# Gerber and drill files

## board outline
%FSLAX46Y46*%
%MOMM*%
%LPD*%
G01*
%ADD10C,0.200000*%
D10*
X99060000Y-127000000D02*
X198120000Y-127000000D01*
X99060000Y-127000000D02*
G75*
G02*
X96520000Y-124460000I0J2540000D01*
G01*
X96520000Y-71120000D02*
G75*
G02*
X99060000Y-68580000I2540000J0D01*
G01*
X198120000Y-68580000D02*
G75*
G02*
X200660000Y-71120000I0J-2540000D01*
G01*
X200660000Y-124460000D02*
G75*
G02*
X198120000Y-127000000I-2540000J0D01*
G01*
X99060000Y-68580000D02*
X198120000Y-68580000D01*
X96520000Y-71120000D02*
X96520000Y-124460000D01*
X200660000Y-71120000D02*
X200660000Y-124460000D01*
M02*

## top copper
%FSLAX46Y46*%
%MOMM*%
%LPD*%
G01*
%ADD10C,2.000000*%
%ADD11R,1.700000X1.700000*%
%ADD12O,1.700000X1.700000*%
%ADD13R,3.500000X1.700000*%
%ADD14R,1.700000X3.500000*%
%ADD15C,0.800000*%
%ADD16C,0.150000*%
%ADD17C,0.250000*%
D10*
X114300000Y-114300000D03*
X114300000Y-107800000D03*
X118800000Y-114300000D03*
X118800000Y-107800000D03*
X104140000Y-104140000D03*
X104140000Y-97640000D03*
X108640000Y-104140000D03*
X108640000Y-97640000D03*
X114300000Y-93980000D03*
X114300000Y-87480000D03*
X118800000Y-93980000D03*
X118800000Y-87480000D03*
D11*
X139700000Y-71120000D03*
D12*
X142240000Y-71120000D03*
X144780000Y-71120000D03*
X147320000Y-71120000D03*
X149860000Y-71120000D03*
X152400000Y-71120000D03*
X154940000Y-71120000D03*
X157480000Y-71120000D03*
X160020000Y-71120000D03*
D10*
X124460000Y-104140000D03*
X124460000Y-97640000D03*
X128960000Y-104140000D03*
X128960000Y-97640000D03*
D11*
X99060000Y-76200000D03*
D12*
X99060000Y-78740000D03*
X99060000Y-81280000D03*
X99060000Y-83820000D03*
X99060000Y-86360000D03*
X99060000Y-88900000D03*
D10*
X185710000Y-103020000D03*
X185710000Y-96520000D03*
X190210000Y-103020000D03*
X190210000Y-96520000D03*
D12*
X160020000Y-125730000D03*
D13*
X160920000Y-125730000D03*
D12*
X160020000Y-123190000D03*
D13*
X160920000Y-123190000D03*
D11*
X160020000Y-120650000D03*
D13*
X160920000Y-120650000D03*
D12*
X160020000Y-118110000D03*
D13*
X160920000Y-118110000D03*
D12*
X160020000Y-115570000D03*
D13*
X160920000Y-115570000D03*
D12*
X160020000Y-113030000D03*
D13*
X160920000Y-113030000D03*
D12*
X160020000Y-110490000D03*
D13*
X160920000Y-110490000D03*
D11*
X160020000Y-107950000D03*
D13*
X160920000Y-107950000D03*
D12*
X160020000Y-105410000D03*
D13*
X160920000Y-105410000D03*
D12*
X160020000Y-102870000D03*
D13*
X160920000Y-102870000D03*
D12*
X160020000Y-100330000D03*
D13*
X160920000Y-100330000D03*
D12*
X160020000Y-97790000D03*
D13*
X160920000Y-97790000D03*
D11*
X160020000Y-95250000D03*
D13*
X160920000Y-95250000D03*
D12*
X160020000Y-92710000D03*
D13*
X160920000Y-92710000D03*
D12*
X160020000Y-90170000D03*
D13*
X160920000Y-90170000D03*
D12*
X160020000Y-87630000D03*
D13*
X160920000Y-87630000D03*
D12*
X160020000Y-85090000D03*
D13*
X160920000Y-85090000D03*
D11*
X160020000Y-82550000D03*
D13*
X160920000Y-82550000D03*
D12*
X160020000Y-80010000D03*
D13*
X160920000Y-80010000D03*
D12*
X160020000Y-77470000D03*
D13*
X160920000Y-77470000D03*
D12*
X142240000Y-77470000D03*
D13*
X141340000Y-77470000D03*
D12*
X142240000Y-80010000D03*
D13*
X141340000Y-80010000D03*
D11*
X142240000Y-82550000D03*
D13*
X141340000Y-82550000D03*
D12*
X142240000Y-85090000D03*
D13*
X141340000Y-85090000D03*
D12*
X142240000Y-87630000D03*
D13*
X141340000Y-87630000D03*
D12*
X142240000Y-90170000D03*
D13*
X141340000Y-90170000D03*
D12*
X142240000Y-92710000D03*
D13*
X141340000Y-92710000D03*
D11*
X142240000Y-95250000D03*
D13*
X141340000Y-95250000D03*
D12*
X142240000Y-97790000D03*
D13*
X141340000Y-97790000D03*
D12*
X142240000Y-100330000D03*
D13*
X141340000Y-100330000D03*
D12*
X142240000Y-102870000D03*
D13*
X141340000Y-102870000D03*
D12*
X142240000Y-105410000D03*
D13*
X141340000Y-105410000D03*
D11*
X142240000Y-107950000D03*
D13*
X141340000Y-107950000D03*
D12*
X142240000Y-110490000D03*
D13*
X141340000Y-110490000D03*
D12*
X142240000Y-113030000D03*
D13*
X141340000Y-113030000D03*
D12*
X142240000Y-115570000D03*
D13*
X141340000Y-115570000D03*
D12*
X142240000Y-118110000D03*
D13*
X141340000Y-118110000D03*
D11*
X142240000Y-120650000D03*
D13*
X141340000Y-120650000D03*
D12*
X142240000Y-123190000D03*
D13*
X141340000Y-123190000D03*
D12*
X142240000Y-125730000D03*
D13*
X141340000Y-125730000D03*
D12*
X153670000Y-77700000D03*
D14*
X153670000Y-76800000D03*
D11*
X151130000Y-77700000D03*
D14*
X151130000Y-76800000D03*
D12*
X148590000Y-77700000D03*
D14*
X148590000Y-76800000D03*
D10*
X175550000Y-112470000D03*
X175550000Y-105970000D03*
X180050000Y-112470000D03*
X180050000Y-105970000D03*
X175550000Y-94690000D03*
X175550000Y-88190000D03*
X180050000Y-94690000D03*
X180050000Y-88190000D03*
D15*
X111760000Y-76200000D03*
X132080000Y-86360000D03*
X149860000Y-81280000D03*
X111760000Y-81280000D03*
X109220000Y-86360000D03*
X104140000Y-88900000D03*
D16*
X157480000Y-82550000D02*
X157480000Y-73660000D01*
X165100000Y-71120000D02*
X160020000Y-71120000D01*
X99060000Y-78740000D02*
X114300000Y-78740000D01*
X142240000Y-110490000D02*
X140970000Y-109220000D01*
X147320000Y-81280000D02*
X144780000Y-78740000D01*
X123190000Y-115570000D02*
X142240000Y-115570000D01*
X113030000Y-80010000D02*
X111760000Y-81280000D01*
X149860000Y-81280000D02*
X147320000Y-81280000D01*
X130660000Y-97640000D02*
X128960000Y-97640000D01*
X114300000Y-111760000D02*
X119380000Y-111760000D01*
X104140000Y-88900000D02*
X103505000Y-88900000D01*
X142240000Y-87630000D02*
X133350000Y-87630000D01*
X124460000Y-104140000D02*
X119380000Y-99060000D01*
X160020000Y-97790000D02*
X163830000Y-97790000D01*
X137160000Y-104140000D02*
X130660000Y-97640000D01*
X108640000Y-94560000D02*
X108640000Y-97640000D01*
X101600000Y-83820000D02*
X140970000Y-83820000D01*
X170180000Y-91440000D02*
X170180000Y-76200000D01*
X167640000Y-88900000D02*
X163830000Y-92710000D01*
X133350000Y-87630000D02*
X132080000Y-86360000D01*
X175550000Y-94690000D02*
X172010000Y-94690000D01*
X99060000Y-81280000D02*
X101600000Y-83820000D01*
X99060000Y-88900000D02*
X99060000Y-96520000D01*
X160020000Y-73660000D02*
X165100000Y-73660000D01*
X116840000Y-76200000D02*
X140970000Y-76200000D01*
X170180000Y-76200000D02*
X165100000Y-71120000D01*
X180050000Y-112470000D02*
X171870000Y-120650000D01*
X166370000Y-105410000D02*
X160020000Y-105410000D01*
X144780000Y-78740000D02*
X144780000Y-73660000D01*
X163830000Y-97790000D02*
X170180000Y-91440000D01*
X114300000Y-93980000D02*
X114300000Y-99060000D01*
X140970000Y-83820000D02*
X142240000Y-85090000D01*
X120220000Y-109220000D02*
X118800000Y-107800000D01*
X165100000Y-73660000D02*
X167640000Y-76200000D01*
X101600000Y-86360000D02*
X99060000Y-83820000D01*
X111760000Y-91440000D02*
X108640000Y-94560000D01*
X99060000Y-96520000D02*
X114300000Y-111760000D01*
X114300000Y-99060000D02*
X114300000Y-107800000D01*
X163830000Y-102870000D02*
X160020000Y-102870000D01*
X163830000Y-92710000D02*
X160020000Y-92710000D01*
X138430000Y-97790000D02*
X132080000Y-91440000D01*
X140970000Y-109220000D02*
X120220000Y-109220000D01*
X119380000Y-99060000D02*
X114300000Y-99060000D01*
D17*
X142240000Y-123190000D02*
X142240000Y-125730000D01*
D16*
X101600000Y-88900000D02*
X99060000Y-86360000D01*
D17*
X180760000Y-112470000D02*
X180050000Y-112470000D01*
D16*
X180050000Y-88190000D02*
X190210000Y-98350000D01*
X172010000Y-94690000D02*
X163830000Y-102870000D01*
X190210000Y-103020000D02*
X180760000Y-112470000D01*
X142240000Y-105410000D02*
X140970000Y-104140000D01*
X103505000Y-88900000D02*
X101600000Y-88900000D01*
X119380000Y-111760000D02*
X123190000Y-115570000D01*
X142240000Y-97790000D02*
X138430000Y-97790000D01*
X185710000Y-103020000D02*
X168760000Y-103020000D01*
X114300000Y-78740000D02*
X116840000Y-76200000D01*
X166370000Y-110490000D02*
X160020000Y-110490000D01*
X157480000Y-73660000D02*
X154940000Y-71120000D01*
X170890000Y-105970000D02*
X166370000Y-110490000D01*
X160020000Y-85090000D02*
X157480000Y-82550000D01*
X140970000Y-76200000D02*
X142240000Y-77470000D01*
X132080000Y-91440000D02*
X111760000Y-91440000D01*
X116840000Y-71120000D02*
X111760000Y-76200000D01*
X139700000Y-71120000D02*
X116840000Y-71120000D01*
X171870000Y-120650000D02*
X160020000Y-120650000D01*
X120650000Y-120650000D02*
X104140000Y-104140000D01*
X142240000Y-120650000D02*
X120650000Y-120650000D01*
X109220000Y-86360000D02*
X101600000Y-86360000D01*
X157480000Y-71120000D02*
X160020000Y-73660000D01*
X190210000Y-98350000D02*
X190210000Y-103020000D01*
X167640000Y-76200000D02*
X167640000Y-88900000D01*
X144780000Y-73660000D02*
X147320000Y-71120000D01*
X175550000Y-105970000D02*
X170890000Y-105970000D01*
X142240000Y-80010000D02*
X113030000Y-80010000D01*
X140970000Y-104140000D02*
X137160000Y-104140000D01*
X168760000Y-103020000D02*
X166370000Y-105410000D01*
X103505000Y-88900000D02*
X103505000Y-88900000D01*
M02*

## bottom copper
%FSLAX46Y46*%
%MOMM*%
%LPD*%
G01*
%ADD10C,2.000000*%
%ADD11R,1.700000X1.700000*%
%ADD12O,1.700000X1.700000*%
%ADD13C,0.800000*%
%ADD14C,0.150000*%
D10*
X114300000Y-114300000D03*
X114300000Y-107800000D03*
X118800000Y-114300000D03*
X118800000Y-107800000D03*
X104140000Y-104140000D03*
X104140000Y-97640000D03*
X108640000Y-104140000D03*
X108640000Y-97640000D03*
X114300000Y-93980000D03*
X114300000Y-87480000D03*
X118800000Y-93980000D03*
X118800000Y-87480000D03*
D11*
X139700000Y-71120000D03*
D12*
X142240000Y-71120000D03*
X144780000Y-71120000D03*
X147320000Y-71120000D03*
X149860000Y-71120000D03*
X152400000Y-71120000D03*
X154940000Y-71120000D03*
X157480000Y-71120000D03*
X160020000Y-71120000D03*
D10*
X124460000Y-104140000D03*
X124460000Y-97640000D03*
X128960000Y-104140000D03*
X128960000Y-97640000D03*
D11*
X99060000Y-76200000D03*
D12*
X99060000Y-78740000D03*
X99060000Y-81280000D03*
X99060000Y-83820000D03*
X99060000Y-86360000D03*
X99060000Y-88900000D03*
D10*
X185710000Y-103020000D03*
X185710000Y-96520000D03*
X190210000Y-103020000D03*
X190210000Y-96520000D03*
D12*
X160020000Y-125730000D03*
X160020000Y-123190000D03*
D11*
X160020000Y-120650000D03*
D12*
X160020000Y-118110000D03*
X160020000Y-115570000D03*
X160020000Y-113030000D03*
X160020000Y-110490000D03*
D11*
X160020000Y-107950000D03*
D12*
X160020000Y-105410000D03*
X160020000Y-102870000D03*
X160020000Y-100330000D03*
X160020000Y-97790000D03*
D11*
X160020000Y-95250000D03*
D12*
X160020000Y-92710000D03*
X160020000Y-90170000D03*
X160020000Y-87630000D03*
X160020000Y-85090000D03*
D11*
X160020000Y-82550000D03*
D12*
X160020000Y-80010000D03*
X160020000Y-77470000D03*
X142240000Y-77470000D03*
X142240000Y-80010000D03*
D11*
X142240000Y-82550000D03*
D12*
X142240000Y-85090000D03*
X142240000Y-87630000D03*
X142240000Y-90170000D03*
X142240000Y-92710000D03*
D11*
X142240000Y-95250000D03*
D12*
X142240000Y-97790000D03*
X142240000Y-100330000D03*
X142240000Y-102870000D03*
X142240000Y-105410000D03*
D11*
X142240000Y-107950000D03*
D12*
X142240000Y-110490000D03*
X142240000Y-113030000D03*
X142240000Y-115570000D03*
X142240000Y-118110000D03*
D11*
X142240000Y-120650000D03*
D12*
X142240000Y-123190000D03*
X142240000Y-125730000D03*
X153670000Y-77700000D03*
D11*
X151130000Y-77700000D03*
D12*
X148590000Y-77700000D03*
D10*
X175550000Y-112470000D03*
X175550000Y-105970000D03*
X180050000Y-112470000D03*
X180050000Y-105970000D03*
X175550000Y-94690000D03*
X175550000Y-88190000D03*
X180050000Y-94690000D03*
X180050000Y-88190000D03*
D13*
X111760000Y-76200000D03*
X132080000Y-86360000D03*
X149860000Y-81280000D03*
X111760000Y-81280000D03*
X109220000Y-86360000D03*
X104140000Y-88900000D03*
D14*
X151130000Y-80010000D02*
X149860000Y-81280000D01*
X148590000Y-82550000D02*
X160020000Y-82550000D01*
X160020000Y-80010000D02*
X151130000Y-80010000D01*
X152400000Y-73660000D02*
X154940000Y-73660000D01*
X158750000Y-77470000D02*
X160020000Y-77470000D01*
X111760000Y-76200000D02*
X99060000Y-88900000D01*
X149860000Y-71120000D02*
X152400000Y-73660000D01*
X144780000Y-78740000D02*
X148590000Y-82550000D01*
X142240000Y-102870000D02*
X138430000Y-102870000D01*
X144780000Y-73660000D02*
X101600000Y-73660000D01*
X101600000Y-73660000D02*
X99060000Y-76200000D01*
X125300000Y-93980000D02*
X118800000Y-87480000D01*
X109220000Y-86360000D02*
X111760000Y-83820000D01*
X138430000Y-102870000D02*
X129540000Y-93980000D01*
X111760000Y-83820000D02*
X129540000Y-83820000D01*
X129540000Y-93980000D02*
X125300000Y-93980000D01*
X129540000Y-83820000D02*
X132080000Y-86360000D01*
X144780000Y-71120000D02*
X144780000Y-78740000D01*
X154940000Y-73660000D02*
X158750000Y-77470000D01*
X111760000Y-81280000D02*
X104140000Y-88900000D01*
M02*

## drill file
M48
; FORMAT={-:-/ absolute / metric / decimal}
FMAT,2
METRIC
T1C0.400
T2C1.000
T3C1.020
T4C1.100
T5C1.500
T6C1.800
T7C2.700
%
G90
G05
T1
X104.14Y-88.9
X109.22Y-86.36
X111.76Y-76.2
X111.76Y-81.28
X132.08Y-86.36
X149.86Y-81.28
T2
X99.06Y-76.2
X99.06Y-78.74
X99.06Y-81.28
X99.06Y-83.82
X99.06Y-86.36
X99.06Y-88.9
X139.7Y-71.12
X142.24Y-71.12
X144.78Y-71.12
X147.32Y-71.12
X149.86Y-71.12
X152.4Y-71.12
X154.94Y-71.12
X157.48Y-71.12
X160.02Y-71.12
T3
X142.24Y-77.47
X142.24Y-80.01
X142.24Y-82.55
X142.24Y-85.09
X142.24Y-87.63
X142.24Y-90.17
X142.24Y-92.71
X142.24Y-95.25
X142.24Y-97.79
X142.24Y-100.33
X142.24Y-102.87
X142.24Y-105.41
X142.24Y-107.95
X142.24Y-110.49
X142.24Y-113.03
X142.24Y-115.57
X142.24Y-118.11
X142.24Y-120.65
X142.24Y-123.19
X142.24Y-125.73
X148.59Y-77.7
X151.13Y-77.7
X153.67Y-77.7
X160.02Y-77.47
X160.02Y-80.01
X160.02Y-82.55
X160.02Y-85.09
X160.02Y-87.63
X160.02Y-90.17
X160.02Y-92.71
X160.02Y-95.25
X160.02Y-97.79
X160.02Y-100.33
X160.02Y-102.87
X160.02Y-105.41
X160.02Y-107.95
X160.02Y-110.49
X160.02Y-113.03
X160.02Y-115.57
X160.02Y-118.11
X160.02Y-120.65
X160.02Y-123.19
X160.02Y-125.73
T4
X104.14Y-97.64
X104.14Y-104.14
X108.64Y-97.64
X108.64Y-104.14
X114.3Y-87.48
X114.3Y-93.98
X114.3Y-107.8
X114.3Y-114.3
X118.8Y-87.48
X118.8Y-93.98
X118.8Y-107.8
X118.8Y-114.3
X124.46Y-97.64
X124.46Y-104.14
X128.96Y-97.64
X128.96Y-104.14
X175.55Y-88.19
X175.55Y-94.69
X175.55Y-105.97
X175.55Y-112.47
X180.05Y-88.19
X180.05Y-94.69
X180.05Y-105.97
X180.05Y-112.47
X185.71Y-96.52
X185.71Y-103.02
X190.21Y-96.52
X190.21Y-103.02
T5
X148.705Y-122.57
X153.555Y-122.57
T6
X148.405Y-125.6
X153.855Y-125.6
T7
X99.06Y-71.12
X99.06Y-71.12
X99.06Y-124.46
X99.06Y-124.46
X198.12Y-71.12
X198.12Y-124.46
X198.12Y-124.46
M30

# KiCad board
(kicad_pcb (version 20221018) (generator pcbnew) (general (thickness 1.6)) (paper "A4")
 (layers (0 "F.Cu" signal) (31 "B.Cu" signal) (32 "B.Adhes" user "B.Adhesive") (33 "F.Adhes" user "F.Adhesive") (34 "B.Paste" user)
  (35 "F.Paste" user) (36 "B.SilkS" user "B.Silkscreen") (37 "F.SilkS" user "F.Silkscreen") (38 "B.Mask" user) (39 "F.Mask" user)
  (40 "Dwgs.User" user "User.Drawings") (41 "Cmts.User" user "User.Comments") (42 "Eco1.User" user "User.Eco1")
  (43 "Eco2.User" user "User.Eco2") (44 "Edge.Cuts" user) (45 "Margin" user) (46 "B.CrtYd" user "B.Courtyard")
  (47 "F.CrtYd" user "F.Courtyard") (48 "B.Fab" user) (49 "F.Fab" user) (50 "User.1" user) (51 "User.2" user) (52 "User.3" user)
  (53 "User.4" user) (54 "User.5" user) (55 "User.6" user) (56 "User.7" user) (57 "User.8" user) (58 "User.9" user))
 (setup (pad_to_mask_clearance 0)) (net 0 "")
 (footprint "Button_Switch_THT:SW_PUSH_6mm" (layer "F.Cu") (at 114.3 114.3 90)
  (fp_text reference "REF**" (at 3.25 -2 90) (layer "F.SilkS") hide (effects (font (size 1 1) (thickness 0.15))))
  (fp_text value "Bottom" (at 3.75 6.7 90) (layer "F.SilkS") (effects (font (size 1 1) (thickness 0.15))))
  (pad "1" thru_hole circle (at 0 0 180) (size 2 2) (drill 1.1) (layers "*.Cu" "*.Mask"))
  (pad "1" thru_hole circle (at 6.5 0 180) (size 2 2) (drill 1.1) (layers "*.Cu" "*.Mask"))
  (pad "2" thru_hole circle (at 0 4.5 180) (size 2 2) (drill 1.1) (layers "*.Cu" "*.Mask"))
  (pad "2" thru_hole circle (at 6.5 4.5 180) (size 2 2) (drill 1.1) (layers "*.Cu" "*.Mask")))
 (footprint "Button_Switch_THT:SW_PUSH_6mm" (layer "F.Cu") (at 104.14 104.14 90)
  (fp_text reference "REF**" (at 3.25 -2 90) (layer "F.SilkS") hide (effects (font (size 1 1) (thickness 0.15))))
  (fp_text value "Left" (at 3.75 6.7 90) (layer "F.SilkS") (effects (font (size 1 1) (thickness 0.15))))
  (pad "1" thru_hole circle (at 0 0 180) (size 2 2) (drill 1.1) (layers "*.Cu" "*.Mask"))
  (pad "1" thru_hole circle (at 6.5 0 180) (size 2 2) (drill 1.1) (layers "*.Cu" "*.Mask"))
  (pad "2" thru_hole circle (at 0 4.5 180) (size 2 2) (drill 1.1) (layers "*.Cu" "*.Mask"))
  (pad "2" thru_hole circle (at 6.5 4.5 180) (size 2 2) (drill 1.1) (layers "*.Cu" "*.Mask")))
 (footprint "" (layer "F.Cu") (at 198.12 71.12)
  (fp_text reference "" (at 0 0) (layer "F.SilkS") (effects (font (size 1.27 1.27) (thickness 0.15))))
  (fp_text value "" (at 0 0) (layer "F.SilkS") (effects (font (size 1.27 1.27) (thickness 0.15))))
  (pad "" np_thru_hole circle (at 0 0) (size 2.7 2.7) (drill 2.7) (layers "F&B.Cu" "*.Mask")))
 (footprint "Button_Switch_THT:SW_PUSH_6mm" (layer "F.Cu") (at 114.3 93.98 90)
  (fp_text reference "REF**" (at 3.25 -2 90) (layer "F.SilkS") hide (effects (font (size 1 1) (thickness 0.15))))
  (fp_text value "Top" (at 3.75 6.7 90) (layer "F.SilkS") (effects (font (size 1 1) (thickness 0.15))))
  (pad "1" thru_hole circle (at 0 0 180) (size 2 2) (drill 1.1) (layers "*.Cu" "*.Mask"))
  (pad "1" thru_hole circle (at 6.5 0 180) (size 2 2) (drill 1.1) (layers "*.Cu" "*.Mask"))
  (pad "2" thru_hole circle (at 0 4.5 180) (size 2 2) (drill 1.1) (layers "*.Cu" "*.Mask"))
  (pad "2" thru_hole circle (at 6.5 4.5 180) (size 2 2) (drill 1.1) (layers "*.Cu" "*.Mask")))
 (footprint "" (layer "F.Cu") (at 99.06 71.12)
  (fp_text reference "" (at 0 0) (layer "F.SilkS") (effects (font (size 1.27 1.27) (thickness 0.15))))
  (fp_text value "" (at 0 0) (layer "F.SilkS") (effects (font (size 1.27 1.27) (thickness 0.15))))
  (pad "" np_thru_hole circle (at 0 0) (size 2.7 2.7) (drill 2.7) (layers "F&B.Cu" "*.Mask")))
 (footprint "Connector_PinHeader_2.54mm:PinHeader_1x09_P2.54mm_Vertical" (layer "F.Cu") (at 139.7 71.12 90)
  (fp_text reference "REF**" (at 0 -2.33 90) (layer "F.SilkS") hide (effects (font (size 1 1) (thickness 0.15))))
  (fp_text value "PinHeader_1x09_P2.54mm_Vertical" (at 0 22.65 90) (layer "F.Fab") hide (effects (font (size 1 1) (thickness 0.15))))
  (pad "1" thru_hole rect (at 0 0 90) (size 1.7 1.7) (drill 1) (layers "*.Cu" "*.Mask"))
  (pad "2" thru_hole oval (at 0 2.54 90) (size 1.7 1.7) (drill 1) (layers "*.Cu" "*.Mask"))
  (pad "3" thru_hole oval (at 0 5.08 90) (size 1.7 1.7) (drill 1) (layers "*.Cu" "*.Mask"))
  (pad "4" thru_hole oval (at 0 7.62 90) (size 1.7 1.7) (drill 1) (layers "*.Cu" "*.Mask"))
  (pad "5" thru_hole oval (at 0 10.16 90) (size 1.7 1.7) (drill 1) (layers "*.Cu" "*.Mask"))
  (pad "6" thru_hole oval (at 0 12.7 90) (size 1.7 1.7) (drill 1) (layers "*.Cu" "*.Mask"))
  (pad "7" thru_hole oval (at 0 15.24 90) (size 1.7 1.7) (drill 1) (layers "*.Cu" "*.Mask"))
  (pad "8" thru_hole oval (at 0 17.78 90) (size 1.7 1.7) (drill 1) (layers "*.Cu" "*.Mask"))
  (pad "9" thru_hole oval (at 0 20.32 90) (size 1.7 1.7) (drill 1) (layers "*.Cu" "*.Mask")))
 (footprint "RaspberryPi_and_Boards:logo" (layer "F.Cu") (at 190.5 76.2)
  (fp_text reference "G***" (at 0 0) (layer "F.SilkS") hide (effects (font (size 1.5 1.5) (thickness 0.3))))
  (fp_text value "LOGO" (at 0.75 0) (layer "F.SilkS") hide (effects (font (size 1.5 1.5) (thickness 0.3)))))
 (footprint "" (layer "F.Cu") (at 198.12 124.46)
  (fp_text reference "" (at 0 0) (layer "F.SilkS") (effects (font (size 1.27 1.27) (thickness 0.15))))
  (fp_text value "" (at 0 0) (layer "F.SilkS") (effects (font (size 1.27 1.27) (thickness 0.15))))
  (pad "" np_thru_hole circle (at 0 0) (size 2.7 2.7) (drill 2.7) (layers "F&B.Cu" "*.Mask")))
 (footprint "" (layer "F.Cu") (at 198.12 124.46)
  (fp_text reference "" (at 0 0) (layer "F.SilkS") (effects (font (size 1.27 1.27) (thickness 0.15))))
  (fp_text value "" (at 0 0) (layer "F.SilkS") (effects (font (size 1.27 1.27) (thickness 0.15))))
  (pad "" np_thru_hole circle (at 0 0) (size 2.7 2.7) (drill 2.7) (layers "F&B.Cu" "*.Mask")))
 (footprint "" (layer "F.Cu") (at 99.06 124.46)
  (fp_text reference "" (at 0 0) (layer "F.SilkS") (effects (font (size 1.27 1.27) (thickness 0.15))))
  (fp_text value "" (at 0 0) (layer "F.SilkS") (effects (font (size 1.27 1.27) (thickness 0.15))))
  (pad "" np_thru_hole circle (at 0 0) (size 2.7 2.7) (drill 2.7) (layers "F&B.Cu" "*.Mask")))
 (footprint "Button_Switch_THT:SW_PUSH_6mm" (layer "F.Cu") (at 124.46 104.14 90)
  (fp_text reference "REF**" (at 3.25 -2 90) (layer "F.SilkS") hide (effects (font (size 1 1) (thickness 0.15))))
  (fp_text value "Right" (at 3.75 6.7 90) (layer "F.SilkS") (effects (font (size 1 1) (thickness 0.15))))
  (pad "1" thru_hole circle (at 0 0 180) (size 2 2) (drill 1.1) (layers "*.Cu" "*.Mask"))
  (pad "1" thru_hole circle (at 6.5 0 180) (size 2 2) (drill 1.1) (layers "*.Cu" "*.Mask"))
  (pad "2" thru_hole circle (at 0 4.5 180) (size 2 2) (drill 1.1) (layers "*.Cu" "*.Mask"))
  (pad "2" thru_hole circle (at 6.5 4.5 180) (size 2 2) (drill 1.1) (layers "*.Cu" "*.Mask")))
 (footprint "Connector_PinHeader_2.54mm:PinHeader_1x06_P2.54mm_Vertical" (layer "F.Cu") (at 99.06 76.2)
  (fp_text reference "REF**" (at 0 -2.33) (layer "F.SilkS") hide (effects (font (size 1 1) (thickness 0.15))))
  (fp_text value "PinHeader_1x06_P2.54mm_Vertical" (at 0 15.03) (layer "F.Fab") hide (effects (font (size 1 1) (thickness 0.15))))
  (pad "1" thru_hole rect (at 0 0) (size 1.7 1.7) (drill 1) (layers "*.Cu" "*.Mask"))
  (pad "2" thru_hole oval (at 0 2.54) (size 1.7 1.7) (drill 1) (layers "*.Cu" "*.Mask"))
  (pad "3" thru_hole oval (at 0 5.08) (size 1.7 1.7) (drill 1) (layers "*.Cu" "*.Mask"))
  (pad "4" thru_hole oval (at 0 7.62) (size 1.7 1.7) (drill 1) (layers "*.Cu" "*.Mask"))
  (pad "5" thru_hole oval (at 0 10.16) (size 1.7 1.7) (drill 1) (layers "*.Cu" "*.Mask"))
  (pad "6" thru_hole oval (at 0 12.7) (size 1.7 1.7) (drill 1) (layers "*.Cu" "*.Mask")))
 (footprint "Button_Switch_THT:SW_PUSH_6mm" (layer "F.Cu") (at 185.71 103.02 90)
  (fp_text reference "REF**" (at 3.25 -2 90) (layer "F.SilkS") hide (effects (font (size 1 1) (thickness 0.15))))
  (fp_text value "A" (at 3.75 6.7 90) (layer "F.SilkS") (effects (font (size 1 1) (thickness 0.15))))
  (pad "1" thru_hole circle (at 0 0 180) (size 2 2) (drill 1.1) (layers "*.Cu" "*.Mask"))
  (pad "1" thru_hole circle (at 6.5 0 180) (size 2 2) (drill 1.1) (layers "*.Cu" "*.Mask"))
  (pad "2" thru_hole circle (at 0 4.5 180) (size 2 2) (drill 1.1) (layers "*.Cu" "*.Mask"))
  (pad "2" thru_hole circle (at 6.5 4.5 180) (size 2 2) (drill 1.1) (layers "*.Cu" "*.Mask")))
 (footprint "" (layer "F.Cu") (at 99.06 124.46)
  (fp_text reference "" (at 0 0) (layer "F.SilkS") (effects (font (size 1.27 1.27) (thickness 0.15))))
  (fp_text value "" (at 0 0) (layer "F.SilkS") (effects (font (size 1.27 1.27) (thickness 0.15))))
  (pad "" np_thru_hole circle (at 0 0) (size 2.7 2.7) (drill 2.7) (layers "F&B.Cu" "*.Mask")))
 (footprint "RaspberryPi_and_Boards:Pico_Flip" (layer "F.Cu") (at 151.13 101.6 180)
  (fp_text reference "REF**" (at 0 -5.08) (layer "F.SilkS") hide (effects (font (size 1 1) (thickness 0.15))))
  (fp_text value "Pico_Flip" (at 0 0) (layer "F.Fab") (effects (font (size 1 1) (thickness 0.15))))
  (pad "" np_thru_hole oval (at -2.725 -24 180) (size 1.8 1.8) (drill 1.8) (layers "*.Cu" "*.Mask"))
  (pad "" np_thru_hole oval (at -2.425 -20.97 180) (size 1.5 1.5) (drill 1.5) (layers "*.Cu" "*.Mask"))
  (pad "" np_thru_hole oval (at 2.425 -20.97 180) (size 1.5 1.5) (drill 1.5) (layers "*.Cu" "*.Mask"))
  (pad "" np_thru_hole oval (at 2.725 -24 180) (size 1.8 1.8) (drill 1.8) (layers "*.Cu" "*.Mask"))
  (pad "1" thru_hole oval (at -8.89 -24.13 180) (size 1.7 1.7) (drill 1.02) (layers "*.Cu" "*.Mask"))
  (pad "1" smd rect (at -8.89 -24.13 180) (size 3.5 1.7) (drill (offset -0.9 0)) (layers "F.Cu" "F.Mask"))
  (pad "2" thru_hole oval (at -8.89 -21.59 180) (size 1.7 1.7) (drill 1.02) (layers "*.Cu" "*.Mask"))
  (pad "2" smd rect (at -8.89 -21.59 180) (size 3.5 1.7) (drill (offset -0.9 0)) (layers "F.Cu" "F.Mask"))
  (pad "3" thru_hole rect (at -8.89 -19.05 180) (size 1.7 1.7) (drill 1.02) (layers "*.Cu" "*.Mask"))
  (pad "3" smd rect (at -8.89 -19.05 180) (size 3.5 1.7) (drill (offset -0.9 0)) (layers "F.Cu" "F.Mask"))
  (pad "4" thru_hole oval (at -8.89 -16.51 180) (size 1.7 1.7) (drill 1.02) (layers "*.Cu" "*.Mask"))
  (pad "4" smd rect (at -8.89 -16.51 180) (size 3.5 1.7) (drill (offset -0.9 0)) (layers "F.Cu" "F.Mask"))
  (pad "5" thru_hole oval (at -8.89 -13.97 180) (size 1.7 1.7) (drill 1.02) (layers "*.Cu" "*.Mask"))
  (pad "5" smd rect (at -8.89 -13.97 180) (size 3.5 1.7) (drill (offset -0.9 0)) (layers "F.Cu" "F.Mask"))
  (pad "6" thru_hole oval (at -8.89 -11.43 180) (size 1.7 1.7) (drill 1.02) (layers "*.Cu" "*.Mask"))
  (pad "6" smd rect (at -8.89 -11.43 180) (size 3.5 1.7) (drill (offset -0.9 0)) (layers "F.Cu" "F.Mask"))
  (pad "7" thru_hole oval (at -8.89 -8.89 180) (size 1.7 1.7) (drill 1.02) (layers "*.Cu" "*.Mask"))
  (pad "7" smd rect (at -8.89 -8.89 180) (size 3.5 1.7) (drill (offset -0.9 0)) (layers "F.Cu" "F.Mask"))
  (pad "8" thru_hole rect (at -8.89 -6.35 180) (size 1.7 1.7) (drill 1.02) (layers "*.Cu" "*.Mask"))
  (pad "8" smd rect (at -8.89 -6.35 180) (size 3.5 1.7) (drill (offset -0.9 0)) (layers "F.Cu" "F.Mask"))
  (pad "9" thru_hole oval (at -8.89 -3.81 180) (size 1.7 1.7) (drill 1.02) (layers "*.Cu" "*.Mask"))
  (pad "9" smd rect (at -8.89 -3.81 180) (size 3.5 1.7) (drill (offset -0.9 0)) (layers "F.Cu" "F.Mask"))
  (pad "10" thru_hole oval (at -8.89 -1.27 180) (size 1.7 1.7) (drill 1.02) (layers "*.Cu" "*.Mask"))
  (pad "10" smd rect (at -8.89 -1.27 180) (size 3.5 1.7) (drill (offset -0.9 0)) (layers "F.Cu" "F.Mask"))
  (pad "11" thru_hole oval (at -8.89 1.27 180) (size 1.7 1.7) (drill 1.02) (layers "*.Cu" "*.Mask"))
  (pad "11" smd rect (at -8.89 1.27 180) (size 3.5 1.7) (drill (offset -0.9 0)) (layers "F.Cu" "F.Mask"))
  (pad "12" thru_hole oval (at -8.89 3.81 180) (size 1.7 1.7) (drill 1.02) (layers "*.Cu" "*.Mask"))
  (pad "12" smd rect (at -8.89 3.81 180) (size 3.5 1.7) (drill (offset -0.9 0)) (layers "F.Cu" "F.Mask"))
  (pad "13" thru_hole rect (at -8.89 6.35 180) (size 1.7 1.7) (drill 1.02) (layers "*.Cu" "*.Mask"))
  (pad "13" smd rect (at -8.89 6.35 180) (size 3.5 1.7) (drill (offset -0.9 0)) (layers "F.Cu" "F.Mask"))
  (pad "14" thru_hole oval (at -8.89 8.89 180) (size 1.7 1.7) (drill 1.02) (layers "*.Cu" "*.Mask"))
  (pad "14" smd rect (at -8.89 8.89 180) (size 3.5 1.7) (drill (offset -0.9 0)) (layers "F.Cu" "F.Mask"))
  (pad "15" thru_hole oval (at -8.89 11.43 180) (size 1.7 1.7) (drill 1.02) (layers "*.Cu" "*.Mask"))
  (pad "15" smd rect (at -8.89 11.43 180) (size 3.5 1.7) (drill (offset -0.9 0)) (layers "F.Cu" "F.Mask"))
  (pad "16" thru_hole oval (at -8.89 13.97 180) (size 1.7 1.7) (drill 1.02) (layers "*.Cu" "*.Mask"))
  (pad "16" smd rect (at -8.89 13.97 180) (size 3.5 1.7) (drill (offset -0.9 0)) (layers "F.Cu" "F.Mask"))
  (pad "17" thru_hole oval (at -8.89 16.51 180) (size 1.7 1.7) (drill 1.02) (layers "*.Cu" "*.Mask"))
  (pad "17" smd rect (at -8.89 16.51 180) (size 3.5 1.7) (drill (offset -0.9 0)) (layers "F.Cu" "F.Mask"))
  (pad "18" thru_hole rect (at -8.89 19.05 180) (size 1.7 1.7) (drill 1.02) (layers "*.Cu" "*.Mask"))
  (pad "18" smd rect (at -8.89 19.05 180) (size 3.5 1.7) (drill (offset -0.9 0)) (layers "F.Cu" "F.Mask"))
  (pad "19" thru_hole oval (at -8.89 21.59 180) (size 1.7 1.7) (drill 1.02) (layers "*.Cu" "*.Mask"))
  (pad "19" smd rect (at -8.89 21.59 180) (size 3.5 1.7) (drill (offset -0.9 0)) (layers "F.Cu" "F.Mask"))
  (pad "20" thru_hole oval (at -8.89 24.13 180) (size 1.7 1.7) (drill 1.02) (layers "*.Cu" "*.Mask"))
  (pad "20" smd rect (at -8.89 24.13 180) (size 3.5 1.7) (drill (offset -0.9 0)) (layers "F.Cu" "F.Mask"))
  (pad "21" thru_hole oval (at 8.89 24.13 180) (size 1.7 1.7) (drill 1.02) (layers "*.Cu" "*.Mask"))
  (pad "21" smd rect (at 8.89 24.13 180) (size 3.5 1.7) (drill (offset 0.9 0)) (layers "F.Cu" "F.Mask"))
  (pad "22" thru_hole oval (at 8.89 21.59 180) (size 1.7 1.7) (drill 1.02) (layers "*.Cu" "*.Mask"))
  (pad "22" smd rect (at 8.89 21.59 180) (size 3.5 1.7) (drill (offset 0.9 0)) (layers "F.Cu" "F.Mask"))
  (pad "23" thru_hole rect (at 8.89 19.05 180) (size 1.7 1.7) (drill 1.02) (layers "*.Cu" "*.Mask"))
  (pad "23" smd rect (at 8.89 19.05 180) (size 3.5 1.7) (drill (offset 0.9 0)) (layers "F.Cu" "F.Mask"))
  (pad "24" thru_hole oval (at 8.89 16.51 180) (size 1.7 1.7) (drill 1.02) (layers "*.Cu" "*.Mask"))
  (pad "24" smd rect (at 8.89 16.51 180) (size 3.5 1.7) (drill (offset 0.9 0)) (layers "F.Cu" "F.Mask"))
  (pad "25" thru_hole oval (at 8.89 13.97 180) (size 1.7 1.7) (drill 1.02) (layers "*.Cu" "*.Mask"))
  (pad "25" smd rect (at 8.89 13.97 180) (size 3.5 1.7) (drill (offset 0.9 0)) (layers "F.Cu" "F.Mask"))
  (pad "26" thru_hole oval (at 8.89 11.43 180) (size 1.7 1.7) (drill 1.02) (layers "*.Cu" "*.Mask"))
  (pad "26" smd rect (at 8.89 11.43 180) (size 3.5 1.7) (drill (offset 0.9 0)) (layers "F.Cu" "F.Mask"))
  (pad "27" thru_hole oval (at 8.89 8.89 180) (size 1.7 1.7) (drill 1.02) (layers "*.Cu" "*.Mask"))
  (pad "27" smd rect (at 8.89 8.89 180) (size 3.5 1.7) (drill (offset 0.9 0)) (layers "F.Cu" "F.Mask"))
  (pad "28" thru_hole rect (at 8.89 6.35 180) (size 1.7 1.7) (drill 1.02) (layers "*.Cu" "*.Mask"))
  (pad "28" smd rect (at 8.89 6.35 180) (size 3.5 1.7) (drill (offset 0.9 0)) (layers "F.Cu" "F.Mask"))
  (pad "29" thru_hole oval (at 8.89 3.81 180) (size 1.7 1.7) (drill 1.02) (layers "*.Cu" "*.Mask"))
  (pad "29" smd rect (at 8.89 3.81 180) (size 3.5 1.7) (drill (offset 0.9 0)) (layers "F.Cu" "F.Mask"))
  (pad "30" thru_hole oval (at 8.89 1.27 180) (size 1.7 1.7) (drill 1.02) (layers "*.Cu" "*.Mask"))
  (pad "30" smd rect (at 8.89 1.27 180) (size 3.5 1.7) (drill (offset 0.9 0)) (layers "F.Cu" "F.Mask"))
  (pad "31" thru_hole oval (at 8.89 -1.27 180) (size 1.7 1.7) (drill 1.02) (layers "*.Cu" "*.Mask"))
  (pad "31" smd rect (at 8.89 -1.27 180) (size 3.5 1.7) (drill (offset 0.9 0)) (layers "F.Cu" "F.Mask"))
  (pad "32" thru_hole oval (at 8.89 -3.81 180) (size 1.7 1.7) (drill 1.02) (layers "*.Cu" "*.Mask"))
  (pad "32" smd rect (at 8.89 -3.81 180) (size 3.5 1.7) (drill (offset 0.9 0)) (layers "F.Cu" "F.Mask"))
  (pad "33" thru_hole rect (at 8.89 -6.35 180) (size 1.7 1.7) (drill 1.02) (layers "*.Cu" "*.Mask"))
  (pad "33" smd rect (at 8.89 -6.35 180) (size 3.5 1.7) (drill (offset 0.9 0)) (layers "F.Cu" "F.Mask"))
  (pad "34" thru_hole oval (at 8.89 -8.89 180) (size 1.7 1.7) (drill 1.02) (layers "*.Cu" "*.Mask"))
  (pad "34" smd rect (at 8.89 -8.89 180) (size 3.5 1.7) (drill (offset 0.9 0)) (layers "F.Cu" "F.Mask"))
  (pad "35" thru_hole oval (at 8.89 -11.43 180) (size 1.7 1.7) (drill 1.02) (layers "*.Cu" "*.Mask"))
  (pad "35" smd rect (at 8.89 -11.43 180) (size 3.5 1.7) (drill (offset 0.9 0)) (layers "F.Cu" "F.Mask"))
  (pad "36" thru_hole oval (at 8.89 -13.97 180) (size 1.7 1.7) (drill 1.02) (layers "*.Cu" "*.Mask"))
  (pad "36" smd rect (at 8.89 -13.97 180) (size 3.5 1.7) (drill (offset 0.9 0)) (layers "F.Cu" "F.Mask"))
  (pad "37" thru_hole oval (at 8.89 -16.51 180) (size 1.7 1.7) (drill 1.02) (layers "*.Cu" "*.Mask"))
  (pad "37" smd rect (at 8.89 -16.51 180) (size 3.5 1.7) (drill (offset 0.9 0)) (layers "F.Cu" "F.Mask"))
  (pad "38" thru_hole rect (at 8.89 -19.05 180) (size 1.7 1.7) (drill 1.02) (layers "*.Cu" "*.Mask"))
  (pad "38" smd rect (at 8.89 -19.05 180) (size 3.5 1.7) (drill (offset 0.9 0)) (layers "F.Cu" "F.Mask"))
  (pad "39" thru_hole oval (at 8.89 -21.59 180) (size 1.7 1.7) (drill 1.02) (layers "*.Cu" "*.Mask"))
  (pad "39" smd rect (at 8.89 -21.59 180) (size 3.5 1.7) (drill (offset 0.9 0)) (layers "F.Cu" "F.Mask"))
  (pad "40" thru_hole oval (at 8.89 -24.13 180) (size 1.7 1.7) (drill 1.02) (layers "*.Cu" "*.Mask"))
  (pad "40" smd rect (at 8.89 -24.13 180) (size 3.5 1.7) (drill (offset 0.9 0)) (layers "F.Cu" "F.Mask"))
  (pad "41" thru_hole oval (at -2.54 23.9 180) (size 1.7 1.7) (drill 1.02) (layers "*.Cu" "*.Mask"))
  (pad "41" smd rect (at -2.54 23.9 270) (size 3.5 1.7) (drill (offset -0.9 0)) (layers "F.Cu" "F.Mask"))
  (pad "42" thru_hole rect (at 0 23.9 180) (size 1.7 1.7) (drill 1.02) (layers "*.Cu" "*.Mask"))
  (pad "42" smd rect (at 0 23.9 270) (size 3.5 1.7) (drill (offset -0.9 0)) (layers "F.Cu" "F.Mask"))
  (pad "43" thru_hole oval (at 2.54 23.9 180) (size 1.7 1.7) (drill 1.02) (layers "*.Cu" "*.Mask"))
  (pad "43" smd rect (at 2.54 23.9 270) (size 3.5 1.7) (drill (offset -0.9 0)) (layers "F.Cu" "F.Mask")))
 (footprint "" (layer "F.Cu") (at 99.06 71.12)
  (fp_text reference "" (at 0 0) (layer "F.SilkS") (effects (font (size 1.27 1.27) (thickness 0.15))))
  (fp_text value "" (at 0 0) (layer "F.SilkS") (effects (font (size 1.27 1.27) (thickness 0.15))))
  (pad "" np_thru_hole circle (at 0 0) (size 2.7 2.7) (drill 2.7) (layers "F&B.Cu" "*.Mask")))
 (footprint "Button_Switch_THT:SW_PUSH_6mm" (layer "F.Cu") (at 175.55 112.47 90)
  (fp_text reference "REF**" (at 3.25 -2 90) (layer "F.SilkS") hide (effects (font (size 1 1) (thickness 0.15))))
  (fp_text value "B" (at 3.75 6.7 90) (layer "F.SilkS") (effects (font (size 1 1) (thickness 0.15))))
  (pad "1" thru_hole circle (at 0 0 180) (size 2 2) (drill 1.1) (layers "*.Cu" "*.Mask"))
  (pad "1" thru_hole circle (at 6.5 0 180) (size 2 2) (drill 1.1) (layers "*.Cu" "*.Mask"))
  (pad "2" thru_hole circle (at 0 4.5 180) (size 2 2) (drill 1.1) (layers "*.Cu" "*.Mask"))
  (pad "2" thru_hole circle (at 6.5 4.5 180) (size 2 2) (drill 1.1) (layers "*.Cu" "*.Mask")))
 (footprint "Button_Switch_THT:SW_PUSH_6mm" (layer "F.Cu") (at 175.55 94.69 90)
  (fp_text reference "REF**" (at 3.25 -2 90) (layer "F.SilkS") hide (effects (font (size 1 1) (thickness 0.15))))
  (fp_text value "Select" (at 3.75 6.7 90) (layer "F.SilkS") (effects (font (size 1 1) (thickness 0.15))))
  (pad "1" thru_hole circle (at 0 0 180) (size 2 2) (drill 1.1) (layers "*.Cu" "*.Mask"))
  (pad "1" thru_hole circle (at 6.5 0 180) (size 2 2) (drill 1.1) (layers "*.Cu" "*.Mask"))
  (pad "2" thru_hole circle (at 0 4.5 180) (size 2 2) (drill 1.1) (layers "*.Cu" "*.Mask"))
  (pad "2" thru_hole circle (at 6.5 4.5 180) (size 2 2) (drill 1.1) (layers "*.Cu" "*.Mask")))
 (gr_line (start 99.06 127) (end 198.12 127) (stroke (width 0.2) (type default)) (layer "Edge.Cuts"))
 (gr_arc (start 99.06 127) (mid 97.263949 126.256051) (end 96.52 124.46) (stroke (width 0.2) (type default)) (layer "Edge.Cuts"))
 (gr_arc (start 96.52 71.12) (mid 97.263949 69.323949) (end 99.06 68.58) (stroke (width 0.2) (type default)) (layer "Edge.Cuts"))
 (gr_arc (start 198.12 68.58) (mid 199.916051 69.323949) (end 200.66 71.12) (stroke (width 0.2) (type default)) (layer "Edge.Cuts"))
 (gr_arc (start 200.66 124.46) (mid 199.916051 126.256051) (end 198.12 127) (stroke (width 0.2) (type default)) (layer "Edge.Cuts"))
 (gr_line (start 99.06 68.58) (end 198.12 68.58) (stroke (width 0.2) (type default)) (layer "Edge.Cuts"))
 (gr_line (start 96.52 71.12) (end 96.52 124.46) (stroke (width 0.2) (type default)) (layer "Edge.Cuts"))
 (gr_line (start 200.66 71.12) (end 200.66 124.46) (stroke (width 0.2) (type default)) (layer "Edge.Cuts"))
 (segment (start 157.48 82.55) (end 157.48 73.66) (width 0.15) (layer "F.Cu") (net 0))
 (segment (start 165.1 71.12) (end 160.02 71.12) (width 0.15) (layer "F.Cu") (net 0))
 (segment (start 99.06 78.74) (end 114.3 78.74) (width 0.15) (layer "F.Cu") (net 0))
 (segment (start 142.24 110.49) (end 140.97 109.22) (width 0.15) (layer "F.Cu") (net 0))
 (segment (start 147.32 81.28) (end 144.78 78.74) (width 0.15) (layer "F.Cu") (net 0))
 (segment (start 123.19 115.57) (end 142.24 115.57) (width 0.15) (layer "F.Cu") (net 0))
 (segment (start 113.03 80.01) (end 111.76 81.28) (width 0.15) (layer "F.Cu") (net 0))
 (segment (start 149.86 81.28) (end 147.32 81.28) (width 0.15) (layer "F.Cu") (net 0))
 (segment (start 130.66 97.64) (end 128.96 97.64) (width 0.15) (layer "F.Cu") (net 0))
 (segment (start 114.3 111.76) (end 119.38 111.76) (width 0.15) (layer "F.Cu") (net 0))
 (segment (start 104.14 88.9) (end 103.505 88.9) (width 0.15) (layer "F.Cu") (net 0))
 (segment (start 142.24 87.63) (end 133.35 87.63) (width 0.15) (layer "F.Cu") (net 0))
 (segment (start 124.46 104.14) (end 119.38 99.06) (width 0.15) (layer "F.Cu") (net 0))
 (segment (start 160.02 97.79) (end 163.83 97.79) (width 0.15) (layer "F.Cu") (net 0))
 (segment (start 137.16 104.14) (end 130.66 97.64) (width 0.15) (layer "F.Cu") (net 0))
 (segment (start 108.64 94.56) (end 108.64 97.64) (width 0.15) (layer "F.Cu") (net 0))
 (segment (start 101.6 83.82) (end 140.97 83.82) (width 0.15) (layer "F.Cu") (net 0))
 (segment (start 170.18 91.44) (end 170.18 76.2) (width 0.15) (layer "F.Cu") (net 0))
 (segment (start 167.64 88.9) (end 163.83 92.71) (width 0.15) (layer "F.Cu") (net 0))
 (segment (start 133.35 87.63) (end 132.08 86.36) (width 0.15) (layer "F.Cu") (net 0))
 (segment (start 175.55 94.69) (end 172.01 94.69) (width 0.15) (layer "F.Cu") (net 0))
 (segment (start 99.06 81.28) (end 101.6 83.82) (width 0.15) (layer "F.Cu") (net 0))
 (segment (start 99.06 88.9) (end 99.06 96.52) (width 0.15) (layer "F.Cu") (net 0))
 (segment (start 160.02 73.66) (end 165.1 73.66) (width 0.15) (layer "F.Cu") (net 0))
 (segment (start 116.84 76.2) (end 140.97 76.2) (width 0.15) (layer "F.Cu") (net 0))
 (segment (start 170.18 76.2) (end 165.1 71.12) (width 0.15) (layer "F.Cu") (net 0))
 (segment (start 180.05 112.47) (end 171.87 120.65) (width 0.15) (layer "F.Cu") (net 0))
 (segment (start 166.37 105.41) (end 160.02 105.41) (width 0.15) (layer "F.Cu") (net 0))
 (segment (start 144.78 78.74) (end 144.78 73.66) (width 0.15) (layer "F.Cu") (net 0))
 (segment (start 163.83 97.79) (end 170.18 91.44) (width 0.15) (layer "F.Cu") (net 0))
 (segment (start 114.3 93.98) (end 114.3 99.06) (width 0.15) (layer "F.Cu") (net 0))
 (segment (start 140.97 83.82) (end 142.24 85.09) (width 0.15) (layer "F.Cu") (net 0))
 (segment (start 120.22 109.22) (end 118.8 107.8) (width 0.15) (layer "F.Cu") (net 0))
 (segment (start 165.1 73.66) (end 167.64 76.2) (width 0.15) (layer "F.Cu") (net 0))
 (segment (start 101.6 86.36) (end 99.06 83.82) (width 0.15) (layer "F.Cu") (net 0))
 (segment (start 111.76 91.44) (end 108.64 94.56) (width 0.15) (layer "F.Cu") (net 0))
 (segment (start 99.06 96.52) (end 114.3 111.76) (width 0.15) (layer "F.Cu") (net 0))
 (segment (start 114.3 99.06) (end 114.3 107.8) (width 0.15) (layer "F.Cu") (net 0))
 (segment (start 163.83 102.87) (end 160.02 102.87) (width 0.15) (layer "F.Cu") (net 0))
 (segment (start 163.83 92.71) (end 160.02 92.71) (width 0.15) (layer "F.Cu") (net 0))
 (segment (start 138.43 97.79) (end 132.08 91.44) (width 0.15) (layer "F.Cu") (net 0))
 (segment (start 140.97 109.22) (end 120.22 109.22) (width 0.15) (layer "F.Cu") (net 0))
 (segment (start 119.38 99.06) (end 114.3 99.06) (width 0.15) (layer "F.Cu") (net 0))
 (segment (start 142.24 123.19) (end 142.24 125.73) (width 0.25) (layer "F.Cu") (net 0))
 (segment (start 101.6 88.9) (end 99.06 86.36) (width 0.15) (layer "F.Cu") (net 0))
 (segment (start 180.76 112.47) (end 180.05 112.47) (width 0.25) (layer "F.Cu") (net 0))
 (segment (start 180.05 88.19) (end 190.21 98.35) (width 0.15) (layer "F.Cu") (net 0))
 (segment (start 172.01 94.69) (end 163.83 102.87) (width 0.15) (layer "F.Cu") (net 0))
 (segment (start 190.21 103.02) (end 180.76 112.47) (width 0.15) (layer "F.Cu") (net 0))
 (segment (start 142.24 105.41) (end 140.97 104.14) (width 0.15) (layer "F.Cu") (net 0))
 (segment (start 103.505 88.9) (end 101.6 88.9) (width 0.15) (layer "F.Cu") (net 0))
 (segment (start 119.38 111.76) (end 123.19 115.57) (width 0.15) (layer "F.Cu") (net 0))
 (segment (start 142.24 97.79) (end 138.43 97.79) (width 0.15) (layer "F.Cu") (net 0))
 (segment (start 185.71 103.02) (end 168.76 103.02) (width 0.15) (layer "F.Cu") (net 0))
 (segment (start 114.3 78.74) (end 116.84 76.2) (width 0.15) (layer "F.Cu") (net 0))
 (segment (start 166.37 110.49) (end 160.02 110.49) (width 0.15) (layer "F.Cu") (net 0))
 (segment (start 157.48 73.66) (end 154.94 71.12) (width 0.15) (layer "F.Cu") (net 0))
 (segment (start 170.89 105.97) (end 166.37 110.49) (width 0.15) (layer "F.Cu") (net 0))
 (segment (start 160.02 85.09) (end 157.48 82.55) (width 0.15) (layer "F.Cu") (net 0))
 (segment (start 140.97 76.2) (end 142.24 77.47) (width 0.15) (layer "F.Cu") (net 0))
 (segment (start 132.08 91.44) (end 111.76 91.44) (width 0.15) (layer "F.Cu") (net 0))
 (segment (start 116.84 71.12) (end 111.76 76.2) (width 0.15) (layer "F.Cu") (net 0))
 (segment (start 139.7 71.12) (end 116.84 71.12) (width 0.15) (layer "F.Cu") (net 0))
 (segment (start 171.87 120.65) (end 160.02 120.65) (width 0.15) (layer "F.Cu") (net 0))
 (segment (start 120.65 120.65) (end 104.14 104.14) (width 0.15) (layer "F.Cu") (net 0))
 (segment (start 142.24 120.65) (end 120.65 120.65) (width 0.15) (layer "F.Cu") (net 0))
 (segment (start 109.22 86.36) (end 101.6 86.36) (width 0.15) (layer "F.Cu") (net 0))
 (segment (start 157.48 71.12) (end 160.02 73.66) (width 0.15) (layer "F.Cu") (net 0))
 (segment (start 190.21 98.35) (end 190.21 103.02) (width 0.15) (layer "F.Cu") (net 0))
 (segment (start 167.64 76.2) (end 167.64 88.9) (width 0.15) (layer "F.Cu") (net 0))
 (segment (start 144.78 73.66) (end 147.32 71.12) (width 0.15) (layer "F.Cu") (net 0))
 (segment (start 175.55 105.97) (end 170.89 105.97) (width 0.15) (layer "F.Cu") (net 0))
 (segment (start 142.24 80.01) (end 113.03 80.01) (width 0.15) (layer "F.Cu") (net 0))
 (segment (start 140.97 104.14) (end 137.16 104.14) (width 0.15) (layer "F.Cu") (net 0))
 (segment (start 168.76 103.02) (end 166.37 105.41) (width 0.15) (layer "F.Cu") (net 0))
 (segment (start 103.505 88.9) (end 103.505 88.9) (width 0.15) (layer "F.Cu") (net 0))
 (via (at 111.76 76.2) (size 0.8) (drill 0.4) (layers "F.Cu" "B.Cu") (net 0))
 (via (at 132.08 86.36) (size 0.8) (drill 0.4) (layers "F.Cu" "B.Cu") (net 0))
 (via (at 149.86 81.28) (size 0.8) (drill 0.4) (layers "F.Cu" "B.Cu") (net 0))
 (via (at 111.76 81.28) (size 0.8) (drill 0.4) (layers "F.Cu" "B.Cu") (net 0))
 (via (at 109.22 86.36) (size 0.8) (drill 0.4) (layers "F.Cu" "B.Cu") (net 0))
 (via (at 104.14 88.9) (size 0.8) (drill 0.4) (layers "F.Cu" "B.Cu") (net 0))
 (segment (start 151.13 80.01) (end 149.86 81.28) (width 0.15) (layer "B.Cu") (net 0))
 (segment (start 148.59 82.55) (end 160.02 82.55) (width 0.15) (layer "B.Cu") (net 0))
 (segment (start 160.02 80.01) (end 151.13 80.01) (width 0.15) (layer "B.Cu") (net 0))
 (segment (start 152.4 73.66) (end 154.94 73.66) (width 0.15) (layer "B.Cu") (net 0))
 (segment (start 158.75 77.47) (end 160.02 77.47) (width 0.15) (layer "B.Cu") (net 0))
 (segment (start 111.76 76.2) (end 99.06 88.9) (width 0.15) (layer "B.Cu") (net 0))
 (segment (start 149.86 71.12) (end 152.4 73.66) (width 0.15) (layer "B.Cu") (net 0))
 (segment (start 144.78 78.74) (end 148.59 82.55) (width 0.15) (layer "B.Cu") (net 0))
 (segment (start 142.24 102.87) (end 138.43 102.87) (width 0.15) (layer "B.Cu") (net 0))
 (segment (start 144.78 73.66) (end 101.6 73.66) (width 0.15) (layer "B.Cu") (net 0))
 (segment (start 101.6 73.66) (end 99.06 76.2) (width 0.15) (layer "B.Cu") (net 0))
 (segment (start 125.3 93.98) (end 118.8 87.48) (width 0.15) (layer "B.Cu") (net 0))
 (segment (start 109.22 86.36) (end 111.76 83.82) (width 0.15) (layer "B.Cu") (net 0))
 (segment (start 138.43 102.87) (end 129.54 93.98) (width 0.15) (layer "B.Cu") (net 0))
 (segment (start 111.76 83.82) (end 129.54 83.82) (width 0.15) (layer "B.Cu") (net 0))
 (segment (start 129.54 93.98) (end 125.3 93.98) (width 0.15) (layer "B.Cu") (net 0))
 (segment (start 129.54 83.82) (end 132.08 86.36) (width 0.15) (layer "B.Cu") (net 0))
 (segment (start 144.78 71.12) (end 144.78 78.74) (width 0.15) (layer "B.Cu") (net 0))
 (segment (start 154.94 73.66) (end 158.75 77.47) (width 0.15) (layer "B.Cu") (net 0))
 (segment (start 111.76 81.28) (end 104.14 88.9) (width 0.15) (layer "B.Cu") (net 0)))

